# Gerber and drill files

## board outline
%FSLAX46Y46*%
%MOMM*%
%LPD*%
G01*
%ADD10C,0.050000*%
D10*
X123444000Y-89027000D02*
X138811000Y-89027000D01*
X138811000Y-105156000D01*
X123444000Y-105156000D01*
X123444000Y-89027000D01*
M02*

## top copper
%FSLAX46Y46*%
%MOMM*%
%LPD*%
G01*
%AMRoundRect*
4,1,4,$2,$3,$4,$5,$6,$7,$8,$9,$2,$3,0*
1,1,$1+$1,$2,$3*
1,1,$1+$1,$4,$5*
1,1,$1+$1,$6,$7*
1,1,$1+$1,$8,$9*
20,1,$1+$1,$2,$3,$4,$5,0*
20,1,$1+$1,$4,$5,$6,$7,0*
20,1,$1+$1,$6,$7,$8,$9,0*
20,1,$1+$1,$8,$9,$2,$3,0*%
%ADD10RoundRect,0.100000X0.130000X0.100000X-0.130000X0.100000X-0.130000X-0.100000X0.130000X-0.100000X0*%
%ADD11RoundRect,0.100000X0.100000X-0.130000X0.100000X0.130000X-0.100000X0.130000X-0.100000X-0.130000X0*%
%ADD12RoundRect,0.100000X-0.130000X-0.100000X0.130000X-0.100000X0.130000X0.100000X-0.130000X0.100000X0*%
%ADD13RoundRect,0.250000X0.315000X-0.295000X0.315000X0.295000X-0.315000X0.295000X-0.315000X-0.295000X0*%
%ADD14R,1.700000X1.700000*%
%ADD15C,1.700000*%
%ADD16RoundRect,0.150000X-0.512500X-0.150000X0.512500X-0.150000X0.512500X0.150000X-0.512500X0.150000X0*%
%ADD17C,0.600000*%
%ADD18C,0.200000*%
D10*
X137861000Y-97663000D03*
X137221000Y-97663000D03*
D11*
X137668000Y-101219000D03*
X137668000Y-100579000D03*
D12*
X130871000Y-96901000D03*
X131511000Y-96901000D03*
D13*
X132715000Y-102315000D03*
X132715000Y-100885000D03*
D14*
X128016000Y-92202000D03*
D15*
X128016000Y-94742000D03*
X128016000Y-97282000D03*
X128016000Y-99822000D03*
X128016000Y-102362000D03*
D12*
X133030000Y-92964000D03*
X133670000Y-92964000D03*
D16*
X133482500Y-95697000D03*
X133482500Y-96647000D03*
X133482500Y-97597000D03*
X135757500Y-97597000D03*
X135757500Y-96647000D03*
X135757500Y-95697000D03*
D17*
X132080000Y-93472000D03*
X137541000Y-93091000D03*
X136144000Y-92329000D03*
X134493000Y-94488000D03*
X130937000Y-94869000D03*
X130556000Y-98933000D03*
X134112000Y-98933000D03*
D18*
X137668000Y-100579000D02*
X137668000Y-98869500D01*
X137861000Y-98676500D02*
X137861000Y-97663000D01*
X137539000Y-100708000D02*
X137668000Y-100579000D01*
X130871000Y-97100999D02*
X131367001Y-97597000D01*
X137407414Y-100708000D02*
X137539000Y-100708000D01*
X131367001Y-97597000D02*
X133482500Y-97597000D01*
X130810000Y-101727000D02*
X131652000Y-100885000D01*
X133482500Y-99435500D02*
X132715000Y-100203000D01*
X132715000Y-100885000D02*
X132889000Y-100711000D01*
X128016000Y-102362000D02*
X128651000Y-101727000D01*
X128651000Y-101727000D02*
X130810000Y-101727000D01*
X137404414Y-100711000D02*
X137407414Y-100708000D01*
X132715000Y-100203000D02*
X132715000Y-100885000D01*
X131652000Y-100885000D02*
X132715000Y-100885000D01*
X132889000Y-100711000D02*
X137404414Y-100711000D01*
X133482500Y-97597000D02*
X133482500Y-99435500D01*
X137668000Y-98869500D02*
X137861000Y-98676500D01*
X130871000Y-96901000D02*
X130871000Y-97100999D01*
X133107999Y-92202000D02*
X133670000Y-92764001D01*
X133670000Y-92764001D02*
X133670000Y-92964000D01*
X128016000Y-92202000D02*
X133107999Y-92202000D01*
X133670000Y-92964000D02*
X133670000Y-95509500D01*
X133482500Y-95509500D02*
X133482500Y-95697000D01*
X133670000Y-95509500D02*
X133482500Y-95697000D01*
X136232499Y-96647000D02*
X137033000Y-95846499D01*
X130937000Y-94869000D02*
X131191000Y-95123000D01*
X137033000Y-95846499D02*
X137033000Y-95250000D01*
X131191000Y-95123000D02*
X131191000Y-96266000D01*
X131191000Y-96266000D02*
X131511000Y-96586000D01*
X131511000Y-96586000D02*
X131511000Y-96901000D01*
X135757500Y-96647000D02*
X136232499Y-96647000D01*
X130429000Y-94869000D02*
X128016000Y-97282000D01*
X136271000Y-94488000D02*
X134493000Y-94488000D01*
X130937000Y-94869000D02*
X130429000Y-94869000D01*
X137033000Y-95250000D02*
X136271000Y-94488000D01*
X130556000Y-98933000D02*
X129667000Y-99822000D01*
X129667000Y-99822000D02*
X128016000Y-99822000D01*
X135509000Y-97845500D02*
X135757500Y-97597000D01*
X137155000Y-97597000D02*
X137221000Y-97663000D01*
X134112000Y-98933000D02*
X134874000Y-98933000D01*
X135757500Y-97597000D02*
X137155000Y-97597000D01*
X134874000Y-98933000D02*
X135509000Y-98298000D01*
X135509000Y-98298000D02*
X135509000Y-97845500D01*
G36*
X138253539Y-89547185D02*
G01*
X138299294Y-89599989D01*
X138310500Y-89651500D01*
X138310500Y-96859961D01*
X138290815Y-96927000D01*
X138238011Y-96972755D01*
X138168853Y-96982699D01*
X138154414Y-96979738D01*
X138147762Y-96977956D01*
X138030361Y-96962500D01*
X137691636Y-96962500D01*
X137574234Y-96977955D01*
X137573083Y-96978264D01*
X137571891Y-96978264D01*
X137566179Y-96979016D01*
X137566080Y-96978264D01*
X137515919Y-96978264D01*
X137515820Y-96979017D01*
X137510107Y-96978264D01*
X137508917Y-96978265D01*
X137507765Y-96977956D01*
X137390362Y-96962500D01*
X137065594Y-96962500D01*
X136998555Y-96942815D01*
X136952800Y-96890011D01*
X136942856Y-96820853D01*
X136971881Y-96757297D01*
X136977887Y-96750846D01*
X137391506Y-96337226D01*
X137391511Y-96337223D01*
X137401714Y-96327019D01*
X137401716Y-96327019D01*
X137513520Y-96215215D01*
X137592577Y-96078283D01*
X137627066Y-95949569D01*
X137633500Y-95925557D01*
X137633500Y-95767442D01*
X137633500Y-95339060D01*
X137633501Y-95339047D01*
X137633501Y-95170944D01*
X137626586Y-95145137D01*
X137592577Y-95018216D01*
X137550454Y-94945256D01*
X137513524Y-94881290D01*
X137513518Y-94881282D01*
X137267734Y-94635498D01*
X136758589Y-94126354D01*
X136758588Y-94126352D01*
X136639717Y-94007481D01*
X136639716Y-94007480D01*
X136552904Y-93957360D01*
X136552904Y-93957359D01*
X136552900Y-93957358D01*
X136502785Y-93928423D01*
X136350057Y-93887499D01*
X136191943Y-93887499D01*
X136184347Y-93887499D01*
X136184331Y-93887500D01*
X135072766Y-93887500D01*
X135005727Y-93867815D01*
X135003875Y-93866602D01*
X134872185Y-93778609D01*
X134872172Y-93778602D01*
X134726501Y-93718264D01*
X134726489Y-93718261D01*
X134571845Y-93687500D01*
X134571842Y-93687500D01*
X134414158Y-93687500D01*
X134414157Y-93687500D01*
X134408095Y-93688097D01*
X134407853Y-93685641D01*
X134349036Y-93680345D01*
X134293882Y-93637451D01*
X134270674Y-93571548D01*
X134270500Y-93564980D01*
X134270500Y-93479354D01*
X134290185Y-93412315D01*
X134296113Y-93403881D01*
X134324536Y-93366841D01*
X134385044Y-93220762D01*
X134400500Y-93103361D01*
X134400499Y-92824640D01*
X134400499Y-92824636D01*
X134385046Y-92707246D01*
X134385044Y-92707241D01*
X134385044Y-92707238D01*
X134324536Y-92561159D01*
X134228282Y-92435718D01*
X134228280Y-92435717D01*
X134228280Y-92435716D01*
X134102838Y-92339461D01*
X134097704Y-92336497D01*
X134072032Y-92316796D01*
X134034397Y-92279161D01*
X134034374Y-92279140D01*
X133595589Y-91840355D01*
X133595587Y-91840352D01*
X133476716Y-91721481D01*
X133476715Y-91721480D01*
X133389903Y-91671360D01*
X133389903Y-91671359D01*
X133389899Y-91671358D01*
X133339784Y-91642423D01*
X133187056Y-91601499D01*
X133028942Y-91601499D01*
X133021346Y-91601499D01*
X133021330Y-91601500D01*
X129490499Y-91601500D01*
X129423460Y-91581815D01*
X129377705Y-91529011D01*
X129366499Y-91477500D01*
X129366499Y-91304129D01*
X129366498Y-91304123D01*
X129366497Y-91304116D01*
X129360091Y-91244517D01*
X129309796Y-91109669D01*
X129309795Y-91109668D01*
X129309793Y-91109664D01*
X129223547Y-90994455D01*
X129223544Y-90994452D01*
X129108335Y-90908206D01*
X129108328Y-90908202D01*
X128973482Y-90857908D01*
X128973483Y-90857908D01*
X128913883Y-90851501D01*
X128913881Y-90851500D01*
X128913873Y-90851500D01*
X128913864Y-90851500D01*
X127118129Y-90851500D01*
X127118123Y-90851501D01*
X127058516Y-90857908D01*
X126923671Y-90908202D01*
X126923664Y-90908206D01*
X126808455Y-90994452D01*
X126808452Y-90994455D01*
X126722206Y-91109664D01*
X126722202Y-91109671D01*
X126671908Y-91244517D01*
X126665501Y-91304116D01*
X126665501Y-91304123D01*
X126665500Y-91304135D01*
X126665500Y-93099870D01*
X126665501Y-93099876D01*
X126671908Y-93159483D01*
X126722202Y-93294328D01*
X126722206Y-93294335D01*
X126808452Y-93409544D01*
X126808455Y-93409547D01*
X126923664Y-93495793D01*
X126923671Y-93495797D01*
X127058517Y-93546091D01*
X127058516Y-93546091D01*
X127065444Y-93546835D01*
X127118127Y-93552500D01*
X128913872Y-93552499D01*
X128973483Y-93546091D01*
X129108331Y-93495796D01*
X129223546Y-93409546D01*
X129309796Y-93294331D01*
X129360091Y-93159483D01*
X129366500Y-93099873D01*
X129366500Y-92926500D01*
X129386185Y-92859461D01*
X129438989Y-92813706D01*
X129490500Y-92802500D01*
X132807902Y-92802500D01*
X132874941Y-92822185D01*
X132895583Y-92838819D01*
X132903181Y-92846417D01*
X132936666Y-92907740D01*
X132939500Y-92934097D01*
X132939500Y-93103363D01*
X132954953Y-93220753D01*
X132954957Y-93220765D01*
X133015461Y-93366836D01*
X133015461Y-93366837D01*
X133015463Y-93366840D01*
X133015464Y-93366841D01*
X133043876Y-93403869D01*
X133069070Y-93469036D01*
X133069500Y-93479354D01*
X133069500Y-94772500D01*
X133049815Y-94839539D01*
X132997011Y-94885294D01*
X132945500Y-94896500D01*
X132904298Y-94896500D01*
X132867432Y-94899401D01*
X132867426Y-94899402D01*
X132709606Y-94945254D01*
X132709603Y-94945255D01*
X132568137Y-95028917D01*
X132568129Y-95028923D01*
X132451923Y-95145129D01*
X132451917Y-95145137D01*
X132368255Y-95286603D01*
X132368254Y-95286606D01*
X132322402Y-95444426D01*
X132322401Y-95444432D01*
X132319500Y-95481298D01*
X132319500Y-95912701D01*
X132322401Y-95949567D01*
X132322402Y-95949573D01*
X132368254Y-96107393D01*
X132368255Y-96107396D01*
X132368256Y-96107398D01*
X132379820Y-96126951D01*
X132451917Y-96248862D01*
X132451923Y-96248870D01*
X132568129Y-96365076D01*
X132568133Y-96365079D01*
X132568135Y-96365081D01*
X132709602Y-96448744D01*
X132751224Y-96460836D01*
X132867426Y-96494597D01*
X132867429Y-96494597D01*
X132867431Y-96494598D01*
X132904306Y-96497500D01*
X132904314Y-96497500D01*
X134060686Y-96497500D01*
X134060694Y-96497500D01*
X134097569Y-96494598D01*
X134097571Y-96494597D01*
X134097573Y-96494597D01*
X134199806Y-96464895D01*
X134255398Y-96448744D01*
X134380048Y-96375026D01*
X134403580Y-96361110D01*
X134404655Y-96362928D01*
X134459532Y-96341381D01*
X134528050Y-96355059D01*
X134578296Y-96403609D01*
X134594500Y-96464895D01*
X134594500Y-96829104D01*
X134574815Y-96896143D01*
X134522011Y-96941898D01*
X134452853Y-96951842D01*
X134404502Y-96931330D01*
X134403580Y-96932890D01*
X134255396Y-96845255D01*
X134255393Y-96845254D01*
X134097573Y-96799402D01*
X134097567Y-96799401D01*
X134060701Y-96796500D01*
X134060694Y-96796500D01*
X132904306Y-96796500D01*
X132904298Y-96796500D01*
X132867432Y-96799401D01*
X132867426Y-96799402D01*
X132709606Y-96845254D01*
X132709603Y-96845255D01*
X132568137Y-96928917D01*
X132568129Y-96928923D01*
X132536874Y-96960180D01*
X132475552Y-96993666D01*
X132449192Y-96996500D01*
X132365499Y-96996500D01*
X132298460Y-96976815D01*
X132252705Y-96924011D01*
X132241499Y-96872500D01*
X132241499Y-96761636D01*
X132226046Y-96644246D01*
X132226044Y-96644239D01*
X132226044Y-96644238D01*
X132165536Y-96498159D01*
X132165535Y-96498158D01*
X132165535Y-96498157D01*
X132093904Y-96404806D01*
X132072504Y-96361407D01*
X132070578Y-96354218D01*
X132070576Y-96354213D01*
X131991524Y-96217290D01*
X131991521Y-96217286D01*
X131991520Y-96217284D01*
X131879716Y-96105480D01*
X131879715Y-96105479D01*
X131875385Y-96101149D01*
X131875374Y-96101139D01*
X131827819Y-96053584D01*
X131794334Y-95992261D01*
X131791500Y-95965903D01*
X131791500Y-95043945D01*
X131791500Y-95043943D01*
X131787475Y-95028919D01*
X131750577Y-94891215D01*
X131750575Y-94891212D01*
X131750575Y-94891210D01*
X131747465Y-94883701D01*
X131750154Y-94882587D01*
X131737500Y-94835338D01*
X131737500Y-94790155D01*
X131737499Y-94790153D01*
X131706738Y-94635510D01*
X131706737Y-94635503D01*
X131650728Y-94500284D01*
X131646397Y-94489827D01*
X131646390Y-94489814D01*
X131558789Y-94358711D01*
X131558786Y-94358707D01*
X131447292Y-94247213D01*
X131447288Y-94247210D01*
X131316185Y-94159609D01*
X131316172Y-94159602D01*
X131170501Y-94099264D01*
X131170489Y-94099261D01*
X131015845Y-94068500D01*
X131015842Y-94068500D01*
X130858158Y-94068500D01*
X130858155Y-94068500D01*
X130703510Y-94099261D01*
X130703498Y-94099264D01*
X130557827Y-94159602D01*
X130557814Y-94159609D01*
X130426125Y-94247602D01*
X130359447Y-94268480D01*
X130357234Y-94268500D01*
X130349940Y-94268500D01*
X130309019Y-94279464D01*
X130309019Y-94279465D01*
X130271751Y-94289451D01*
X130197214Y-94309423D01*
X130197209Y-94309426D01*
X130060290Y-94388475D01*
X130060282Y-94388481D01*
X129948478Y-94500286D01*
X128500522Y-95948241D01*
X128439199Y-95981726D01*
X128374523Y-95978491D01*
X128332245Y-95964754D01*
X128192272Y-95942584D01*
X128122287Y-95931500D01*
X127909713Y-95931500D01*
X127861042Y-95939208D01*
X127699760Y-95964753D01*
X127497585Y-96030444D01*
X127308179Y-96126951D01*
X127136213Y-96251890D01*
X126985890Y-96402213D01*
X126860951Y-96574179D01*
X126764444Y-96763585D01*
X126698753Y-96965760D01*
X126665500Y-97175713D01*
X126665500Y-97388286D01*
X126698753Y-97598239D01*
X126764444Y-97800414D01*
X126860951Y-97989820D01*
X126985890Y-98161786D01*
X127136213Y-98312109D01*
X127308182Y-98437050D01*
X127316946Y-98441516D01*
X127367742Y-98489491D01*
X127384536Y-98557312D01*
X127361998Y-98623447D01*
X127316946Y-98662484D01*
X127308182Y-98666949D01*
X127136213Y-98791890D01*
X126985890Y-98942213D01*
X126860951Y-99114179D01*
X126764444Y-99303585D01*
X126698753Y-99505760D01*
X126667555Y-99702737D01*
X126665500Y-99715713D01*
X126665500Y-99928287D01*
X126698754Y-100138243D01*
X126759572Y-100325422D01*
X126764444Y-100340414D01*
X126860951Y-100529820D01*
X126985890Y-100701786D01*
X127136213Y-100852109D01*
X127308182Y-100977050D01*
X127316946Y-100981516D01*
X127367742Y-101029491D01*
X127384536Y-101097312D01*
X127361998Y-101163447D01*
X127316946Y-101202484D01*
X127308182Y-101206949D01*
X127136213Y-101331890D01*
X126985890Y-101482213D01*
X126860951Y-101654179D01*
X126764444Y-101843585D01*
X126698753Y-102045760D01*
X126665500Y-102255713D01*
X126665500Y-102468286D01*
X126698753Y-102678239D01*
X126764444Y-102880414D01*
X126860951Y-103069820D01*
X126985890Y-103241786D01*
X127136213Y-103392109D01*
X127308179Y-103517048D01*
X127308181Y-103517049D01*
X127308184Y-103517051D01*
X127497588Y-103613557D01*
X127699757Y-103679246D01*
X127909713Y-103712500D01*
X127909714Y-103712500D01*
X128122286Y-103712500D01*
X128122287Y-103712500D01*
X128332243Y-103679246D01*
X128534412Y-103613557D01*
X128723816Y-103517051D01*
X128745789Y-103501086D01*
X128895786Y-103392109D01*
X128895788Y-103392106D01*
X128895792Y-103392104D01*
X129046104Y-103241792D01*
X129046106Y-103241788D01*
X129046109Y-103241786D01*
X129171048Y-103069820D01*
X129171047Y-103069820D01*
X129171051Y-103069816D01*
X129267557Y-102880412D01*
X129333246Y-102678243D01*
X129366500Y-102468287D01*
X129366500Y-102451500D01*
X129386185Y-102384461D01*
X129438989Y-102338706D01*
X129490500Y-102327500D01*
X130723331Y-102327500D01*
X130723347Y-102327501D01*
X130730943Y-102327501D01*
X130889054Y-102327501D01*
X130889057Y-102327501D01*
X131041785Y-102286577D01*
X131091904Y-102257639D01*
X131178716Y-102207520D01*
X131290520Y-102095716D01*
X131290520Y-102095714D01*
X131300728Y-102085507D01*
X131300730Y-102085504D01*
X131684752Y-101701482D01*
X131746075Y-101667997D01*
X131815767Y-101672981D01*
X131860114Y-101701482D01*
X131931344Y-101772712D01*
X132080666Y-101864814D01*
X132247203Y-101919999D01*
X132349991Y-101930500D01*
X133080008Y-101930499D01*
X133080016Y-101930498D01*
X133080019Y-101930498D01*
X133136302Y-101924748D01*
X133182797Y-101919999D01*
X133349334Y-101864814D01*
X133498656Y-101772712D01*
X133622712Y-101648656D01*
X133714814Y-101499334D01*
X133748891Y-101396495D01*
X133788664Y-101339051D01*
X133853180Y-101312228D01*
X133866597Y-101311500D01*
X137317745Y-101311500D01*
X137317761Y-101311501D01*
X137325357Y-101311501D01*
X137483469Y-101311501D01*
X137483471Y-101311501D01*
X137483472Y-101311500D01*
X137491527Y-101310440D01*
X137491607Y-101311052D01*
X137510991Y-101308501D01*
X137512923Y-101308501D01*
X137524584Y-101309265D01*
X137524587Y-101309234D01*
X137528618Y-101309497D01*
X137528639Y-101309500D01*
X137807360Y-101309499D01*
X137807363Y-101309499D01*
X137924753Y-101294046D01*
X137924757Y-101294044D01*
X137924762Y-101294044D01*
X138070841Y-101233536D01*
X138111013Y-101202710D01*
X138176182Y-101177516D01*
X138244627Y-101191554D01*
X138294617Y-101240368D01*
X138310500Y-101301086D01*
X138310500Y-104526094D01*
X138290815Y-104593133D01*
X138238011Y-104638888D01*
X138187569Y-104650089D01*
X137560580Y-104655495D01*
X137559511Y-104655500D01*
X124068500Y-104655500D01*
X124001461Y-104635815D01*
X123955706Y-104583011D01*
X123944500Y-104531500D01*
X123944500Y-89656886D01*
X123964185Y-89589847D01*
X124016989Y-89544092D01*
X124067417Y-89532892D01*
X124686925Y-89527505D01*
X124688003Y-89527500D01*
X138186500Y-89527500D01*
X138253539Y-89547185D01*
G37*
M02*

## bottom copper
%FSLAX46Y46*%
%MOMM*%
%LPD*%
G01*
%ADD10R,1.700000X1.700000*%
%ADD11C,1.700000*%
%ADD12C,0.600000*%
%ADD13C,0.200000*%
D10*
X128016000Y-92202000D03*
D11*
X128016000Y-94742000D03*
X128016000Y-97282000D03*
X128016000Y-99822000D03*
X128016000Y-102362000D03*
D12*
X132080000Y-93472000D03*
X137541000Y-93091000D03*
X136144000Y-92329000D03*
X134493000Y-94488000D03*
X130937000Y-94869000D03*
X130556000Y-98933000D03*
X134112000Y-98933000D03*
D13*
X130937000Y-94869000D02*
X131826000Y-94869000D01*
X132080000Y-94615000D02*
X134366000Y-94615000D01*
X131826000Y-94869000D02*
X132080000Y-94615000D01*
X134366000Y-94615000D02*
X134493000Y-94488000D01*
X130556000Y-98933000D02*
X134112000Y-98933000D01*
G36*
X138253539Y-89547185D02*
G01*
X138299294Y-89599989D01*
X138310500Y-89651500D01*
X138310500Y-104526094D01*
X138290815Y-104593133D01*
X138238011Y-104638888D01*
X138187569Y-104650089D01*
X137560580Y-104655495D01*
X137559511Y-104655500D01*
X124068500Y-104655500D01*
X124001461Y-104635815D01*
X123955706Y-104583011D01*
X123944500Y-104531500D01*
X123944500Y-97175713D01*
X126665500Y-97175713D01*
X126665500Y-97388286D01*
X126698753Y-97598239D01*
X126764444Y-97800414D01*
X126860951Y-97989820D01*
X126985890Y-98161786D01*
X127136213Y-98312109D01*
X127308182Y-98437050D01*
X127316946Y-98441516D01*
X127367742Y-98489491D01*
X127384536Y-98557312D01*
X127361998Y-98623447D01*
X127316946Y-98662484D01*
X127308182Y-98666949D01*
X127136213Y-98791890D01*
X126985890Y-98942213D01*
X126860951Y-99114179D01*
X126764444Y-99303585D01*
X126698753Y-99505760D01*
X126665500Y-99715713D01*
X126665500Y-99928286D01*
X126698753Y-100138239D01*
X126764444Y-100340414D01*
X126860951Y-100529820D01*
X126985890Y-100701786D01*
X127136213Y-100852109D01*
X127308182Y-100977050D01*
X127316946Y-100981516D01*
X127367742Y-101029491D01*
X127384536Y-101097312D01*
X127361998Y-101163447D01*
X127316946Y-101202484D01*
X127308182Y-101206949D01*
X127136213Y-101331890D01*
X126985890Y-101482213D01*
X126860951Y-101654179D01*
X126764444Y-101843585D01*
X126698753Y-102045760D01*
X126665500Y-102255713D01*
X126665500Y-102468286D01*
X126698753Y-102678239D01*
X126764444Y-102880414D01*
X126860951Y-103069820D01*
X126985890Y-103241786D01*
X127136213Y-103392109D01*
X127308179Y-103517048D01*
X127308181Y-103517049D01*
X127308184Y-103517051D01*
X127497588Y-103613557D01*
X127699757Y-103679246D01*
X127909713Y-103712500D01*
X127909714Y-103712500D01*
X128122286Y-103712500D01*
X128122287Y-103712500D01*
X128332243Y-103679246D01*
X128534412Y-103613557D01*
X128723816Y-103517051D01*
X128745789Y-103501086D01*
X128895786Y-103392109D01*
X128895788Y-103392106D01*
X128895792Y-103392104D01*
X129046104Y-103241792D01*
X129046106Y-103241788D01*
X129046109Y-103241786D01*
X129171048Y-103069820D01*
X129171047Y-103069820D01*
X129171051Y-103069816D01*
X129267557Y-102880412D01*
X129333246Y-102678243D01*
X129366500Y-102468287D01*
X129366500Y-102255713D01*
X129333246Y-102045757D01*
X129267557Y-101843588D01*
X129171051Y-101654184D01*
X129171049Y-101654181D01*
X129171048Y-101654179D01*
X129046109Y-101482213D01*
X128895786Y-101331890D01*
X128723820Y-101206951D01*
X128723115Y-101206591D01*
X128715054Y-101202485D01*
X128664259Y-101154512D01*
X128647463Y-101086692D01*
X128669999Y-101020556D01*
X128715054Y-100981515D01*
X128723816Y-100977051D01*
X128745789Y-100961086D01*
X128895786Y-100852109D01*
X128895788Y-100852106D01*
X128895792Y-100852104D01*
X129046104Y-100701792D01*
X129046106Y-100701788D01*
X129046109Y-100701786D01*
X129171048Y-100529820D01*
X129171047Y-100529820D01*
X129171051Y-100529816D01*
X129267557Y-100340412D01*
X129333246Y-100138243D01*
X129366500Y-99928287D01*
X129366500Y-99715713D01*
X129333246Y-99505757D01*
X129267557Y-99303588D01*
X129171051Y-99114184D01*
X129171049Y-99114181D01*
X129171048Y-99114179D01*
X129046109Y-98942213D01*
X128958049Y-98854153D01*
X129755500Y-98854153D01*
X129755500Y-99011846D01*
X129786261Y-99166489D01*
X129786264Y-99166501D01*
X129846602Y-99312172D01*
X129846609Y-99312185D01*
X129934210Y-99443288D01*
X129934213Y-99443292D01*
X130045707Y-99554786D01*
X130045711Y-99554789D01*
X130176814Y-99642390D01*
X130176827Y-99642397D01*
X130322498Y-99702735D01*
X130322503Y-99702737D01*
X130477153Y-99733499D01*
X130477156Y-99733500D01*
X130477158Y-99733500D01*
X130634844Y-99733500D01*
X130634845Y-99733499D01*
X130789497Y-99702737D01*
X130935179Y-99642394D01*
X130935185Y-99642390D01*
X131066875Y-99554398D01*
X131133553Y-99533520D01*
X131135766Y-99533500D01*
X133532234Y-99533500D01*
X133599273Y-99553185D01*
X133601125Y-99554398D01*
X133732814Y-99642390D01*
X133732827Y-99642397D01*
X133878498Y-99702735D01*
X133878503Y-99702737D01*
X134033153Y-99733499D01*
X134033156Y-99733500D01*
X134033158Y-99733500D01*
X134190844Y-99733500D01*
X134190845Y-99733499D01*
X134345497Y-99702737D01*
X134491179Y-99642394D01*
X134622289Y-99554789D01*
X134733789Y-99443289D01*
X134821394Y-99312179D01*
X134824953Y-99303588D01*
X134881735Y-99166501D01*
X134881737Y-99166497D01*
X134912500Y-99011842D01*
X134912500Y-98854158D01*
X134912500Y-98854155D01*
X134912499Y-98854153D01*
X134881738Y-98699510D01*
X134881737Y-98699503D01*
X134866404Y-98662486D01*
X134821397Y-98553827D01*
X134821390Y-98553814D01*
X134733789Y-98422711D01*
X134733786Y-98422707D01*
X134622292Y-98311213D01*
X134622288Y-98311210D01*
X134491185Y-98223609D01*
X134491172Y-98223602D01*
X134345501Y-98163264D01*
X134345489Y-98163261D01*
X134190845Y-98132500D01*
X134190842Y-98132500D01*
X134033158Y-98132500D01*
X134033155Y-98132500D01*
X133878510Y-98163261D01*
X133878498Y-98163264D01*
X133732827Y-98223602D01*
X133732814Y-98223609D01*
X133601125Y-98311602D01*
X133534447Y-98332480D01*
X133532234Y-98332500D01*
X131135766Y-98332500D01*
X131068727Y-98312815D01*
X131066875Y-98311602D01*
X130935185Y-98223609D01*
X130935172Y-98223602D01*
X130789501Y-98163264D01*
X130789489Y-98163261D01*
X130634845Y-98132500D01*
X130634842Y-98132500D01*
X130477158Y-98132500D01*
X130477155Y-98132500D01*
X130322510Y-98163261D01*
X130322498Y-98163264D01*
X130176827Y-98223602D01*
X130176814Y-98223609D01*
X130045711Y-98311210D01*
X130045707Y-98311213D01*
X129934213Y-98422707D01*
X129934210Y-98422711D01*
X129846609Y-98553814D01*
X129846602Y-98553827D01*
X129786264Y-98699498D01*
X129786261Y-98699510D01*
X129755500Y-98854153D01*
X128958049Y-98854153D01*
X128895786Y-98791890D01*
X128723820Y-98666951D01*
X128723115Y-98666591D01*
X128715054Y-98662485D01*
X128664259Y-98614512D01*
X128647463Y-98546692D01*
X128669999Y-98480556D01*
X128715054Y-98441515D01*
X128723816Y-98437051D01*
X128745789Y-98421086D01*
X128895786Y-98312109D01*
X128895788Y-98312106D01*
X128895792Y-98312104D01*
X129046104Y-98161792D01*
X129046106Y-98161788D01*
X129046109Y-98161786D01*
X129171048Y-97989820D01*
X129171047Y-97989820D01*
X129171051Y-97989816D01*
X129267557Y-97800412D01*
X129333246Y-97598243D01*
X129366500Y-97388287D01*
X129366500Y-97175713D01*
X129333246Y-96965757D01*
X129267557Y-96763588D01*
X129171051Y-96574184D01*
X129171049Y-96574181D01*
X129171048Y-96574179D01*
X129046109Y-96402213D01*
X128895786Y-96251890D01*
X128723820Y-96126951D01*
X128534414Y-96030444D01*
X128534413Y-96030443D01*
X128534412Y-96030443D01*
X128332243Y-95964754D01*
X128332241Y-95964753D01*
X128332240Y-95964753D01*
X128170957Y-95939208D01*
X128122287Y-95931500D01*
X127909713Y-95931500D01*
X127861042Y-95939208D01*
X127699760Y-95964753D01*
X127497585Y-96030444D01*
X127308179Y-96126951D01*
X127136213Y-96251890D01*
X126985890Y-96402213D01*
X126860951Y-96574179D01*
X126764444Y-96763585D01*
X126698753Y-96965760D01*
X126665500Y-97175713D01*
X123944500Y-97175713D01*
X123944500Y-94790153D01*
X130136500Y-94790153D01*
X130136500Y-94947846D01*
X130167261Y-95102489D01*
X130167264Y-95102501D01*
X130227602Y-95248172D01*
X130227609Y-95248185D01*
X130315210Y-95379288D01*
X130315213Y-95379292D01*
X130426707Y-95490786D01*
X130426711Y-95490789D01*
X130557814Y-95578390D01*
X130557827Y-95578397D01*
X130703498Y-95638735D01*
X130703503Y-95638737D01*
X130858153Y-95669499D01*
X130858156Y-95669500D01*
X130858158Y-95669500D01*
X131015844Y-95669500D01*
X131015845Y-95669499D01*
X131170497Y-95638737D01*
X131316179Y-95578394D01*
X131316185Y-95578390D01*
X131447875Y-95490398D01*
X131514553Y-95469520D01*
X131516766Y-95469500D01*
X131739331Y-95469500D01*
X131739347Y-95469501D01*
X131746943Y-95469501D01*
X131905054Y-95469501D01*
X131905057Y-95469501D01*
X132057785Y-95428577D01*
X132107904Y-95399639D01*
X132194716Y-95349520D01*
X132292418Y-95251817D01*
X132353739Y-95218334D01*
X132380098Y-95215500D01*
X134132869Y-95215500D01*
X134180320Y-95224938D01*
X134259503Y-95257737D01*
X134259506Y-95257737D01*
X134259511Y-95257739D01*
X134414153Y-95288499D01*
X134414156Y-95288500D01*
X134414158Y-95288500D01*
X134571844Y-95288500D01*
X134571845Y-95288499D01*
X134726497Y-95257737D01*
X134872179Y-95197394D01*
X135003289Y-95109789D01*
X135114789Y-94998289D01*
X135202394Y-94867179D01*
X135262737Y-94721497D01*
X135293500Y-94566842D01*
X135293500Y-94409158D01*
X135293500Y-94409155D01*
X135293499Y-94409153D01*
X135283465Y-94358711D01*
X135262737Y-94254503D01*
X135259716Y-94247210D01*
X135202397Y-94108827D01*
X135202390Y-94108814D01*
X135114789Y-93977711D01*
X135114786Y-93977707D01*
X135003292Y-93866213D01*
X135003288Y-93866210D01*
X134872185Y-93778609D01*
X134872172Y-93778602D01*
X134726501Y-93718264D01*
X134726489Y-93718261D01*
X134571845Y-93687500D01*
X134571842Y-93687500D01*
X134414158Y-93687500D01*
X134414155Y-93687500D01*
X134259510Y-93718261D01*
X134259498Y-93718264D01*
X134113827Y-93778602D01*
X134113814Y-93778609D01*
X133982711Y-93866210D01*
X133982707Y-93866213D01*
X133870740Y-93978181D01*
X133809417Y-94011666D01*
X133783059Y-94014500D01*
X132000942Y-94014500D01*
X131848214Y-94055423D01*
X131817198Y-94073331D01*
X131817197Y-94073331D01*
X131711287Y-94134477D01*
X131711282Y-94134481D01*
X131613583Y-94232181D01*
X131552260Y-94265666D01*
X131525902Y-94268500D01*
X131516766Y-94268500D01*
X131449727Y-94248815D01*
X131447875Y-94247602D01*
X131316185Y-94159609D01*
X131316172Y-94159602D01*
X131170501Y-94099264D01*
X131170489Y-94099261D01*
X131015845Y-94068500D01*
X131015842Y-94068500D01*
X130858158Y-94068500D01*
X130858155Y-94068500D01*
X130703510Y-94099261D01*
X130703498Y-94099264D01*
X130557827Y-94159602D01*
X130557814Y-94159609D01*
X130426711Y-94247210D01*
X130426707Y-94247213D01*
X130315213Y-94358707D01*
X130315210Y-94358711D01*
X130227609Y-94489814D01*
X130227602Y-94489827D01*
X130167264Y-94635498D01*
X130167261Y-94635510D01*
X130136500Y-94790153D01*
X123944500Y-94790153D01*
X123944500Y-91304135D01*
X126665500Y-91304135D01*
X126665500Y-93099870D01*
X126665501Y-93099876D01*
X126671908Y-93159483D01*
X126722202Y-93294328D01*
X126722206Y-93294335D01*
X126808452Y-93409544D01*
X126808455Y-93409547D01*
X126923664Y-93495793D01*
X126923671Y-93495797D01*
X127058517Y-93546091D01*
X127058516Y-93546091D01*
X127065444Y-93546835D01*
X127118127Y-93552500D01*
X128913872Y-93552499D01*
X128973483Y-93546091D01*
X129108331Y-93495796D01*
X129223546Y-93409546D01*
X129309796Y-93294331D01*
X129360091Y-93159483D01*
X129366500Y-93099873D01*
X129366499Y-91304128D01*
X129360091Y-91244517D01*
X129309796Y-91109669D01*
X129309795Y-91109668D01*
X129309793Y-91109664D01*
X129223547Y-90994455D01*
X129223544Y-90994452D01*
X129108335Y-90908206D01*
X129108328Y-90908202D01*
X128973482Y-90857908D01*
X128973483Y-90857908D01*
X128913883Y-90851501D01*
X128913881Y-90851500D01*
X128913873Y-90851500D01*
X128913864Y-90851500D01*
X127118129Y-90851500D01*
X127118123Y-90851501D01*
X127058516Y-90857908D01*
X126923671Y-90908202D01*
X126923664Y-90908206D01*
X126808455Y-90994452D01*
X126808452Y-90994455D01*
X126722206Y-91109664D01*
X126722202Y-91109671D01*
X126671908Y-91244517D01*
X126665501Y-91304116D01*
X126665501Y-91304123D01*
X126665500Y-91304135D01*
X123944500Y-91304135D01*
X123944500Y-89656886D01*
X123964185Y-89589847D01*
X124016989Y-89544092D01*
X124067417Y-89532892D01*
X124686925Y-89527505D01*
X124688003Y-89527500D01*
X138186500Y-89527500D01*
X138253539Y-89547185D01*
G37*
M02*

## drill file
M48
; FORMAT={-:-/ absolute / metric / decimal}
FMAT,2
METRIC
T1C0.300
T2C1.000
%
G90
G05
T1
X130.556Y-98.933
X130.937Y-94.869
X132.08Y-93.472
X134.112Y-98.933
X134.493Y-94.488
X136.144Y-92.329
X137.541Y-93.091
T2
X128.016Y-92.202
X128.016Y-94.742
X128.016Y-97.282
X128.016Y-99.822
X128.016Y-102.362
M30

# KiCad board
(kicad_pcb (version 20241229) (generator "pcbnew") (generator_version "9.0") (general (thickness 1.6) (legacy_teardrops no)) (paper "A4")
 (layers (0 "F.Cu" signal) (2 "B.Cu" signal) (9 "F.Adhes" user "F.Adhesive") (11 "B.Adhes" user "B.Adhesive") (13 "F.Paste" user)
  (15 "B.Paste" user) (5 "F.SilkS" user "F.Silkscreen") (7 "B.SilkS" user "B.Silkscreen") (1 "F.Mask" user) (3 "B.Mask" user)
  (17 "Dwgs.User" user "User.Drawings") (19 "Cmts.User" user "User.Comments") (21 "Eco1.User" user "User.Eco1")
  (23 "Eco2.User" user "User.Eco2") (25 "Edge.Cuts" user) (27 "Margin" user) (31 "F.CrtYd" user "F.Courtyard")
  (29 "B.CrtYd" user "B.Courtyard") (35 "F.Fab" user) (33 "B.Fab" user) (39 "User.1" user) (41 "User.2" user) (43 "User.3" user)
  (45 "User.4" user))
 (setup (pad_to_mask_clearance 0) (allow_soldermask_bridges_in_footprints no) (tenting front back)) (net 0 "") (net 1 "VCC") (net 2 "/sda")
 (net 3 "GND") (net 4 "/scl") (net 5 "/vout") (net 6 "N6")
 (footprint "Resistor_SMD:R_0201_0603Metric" (layer "F.Cu") (at 137.541 97.663 180)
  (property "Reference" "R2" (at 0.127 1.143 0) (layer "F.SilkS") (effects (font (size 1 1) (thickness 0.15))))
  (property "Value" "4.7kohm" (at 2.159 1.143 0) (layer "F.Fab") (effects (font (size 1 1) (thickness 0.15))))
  (pad "" smd roundrect (at -0.345 0 180) (size 0.318 0.36) (layers "F.Paste") (roundrect_rratio 0.25))
  (pad "" smd roundrect (at 0.345 0 180) (size 0.318 0.36) (layers "F.Paste") (roundrect_rratio 0.25))
  (pad "1" smd roundrect (at -0.32 0 180) (size 0.46 0.4) (layers "F.Cu" "F.Mask") (roundrect_rratio 0.25) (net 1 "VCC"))
  (pad "2" smd roundrect (at 0.32 0 180) (size 0.46 0.4) (layers "F.Cu" "F.Mask") (roundrect_rratio 0.25) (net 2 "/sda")))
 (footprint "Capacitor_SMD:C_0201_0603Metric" (layer "F.Cu") (at 137.668 100.899 90)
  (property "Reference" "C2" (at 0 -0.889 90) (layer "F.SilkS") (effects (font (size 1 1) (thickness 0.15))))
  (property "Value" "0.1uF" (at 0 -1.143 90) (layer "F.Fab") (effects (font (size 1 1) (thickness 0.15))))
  (pad "" smd roundrect (at -0.345 0 90) (size 0.318 0.36) (layers "F.Paste") (roundrect_rratio 0.25))
  (pad "" smd roundrect (at 0.345 0 90) (size 0.318 0.36) (layers "F.Paste") (roundrect_rratio 0.25))
  (pad "1" smd roundrect (at -0.32 0 90) (size 0.46 0.4) (layers "F.Cu" "F.Mask") (roundrect_rratio 0.25) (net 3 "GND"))
  (pad "2" smd roundrect (at 0.32 0 90) (size 0.46 0.4) (layers "F.Cu" "F.Mask") (roundrect_rratio 0.25) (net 1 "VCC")))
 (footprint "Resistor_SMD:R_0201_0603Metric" (layer "F.Cu") (at 131.191 96.901)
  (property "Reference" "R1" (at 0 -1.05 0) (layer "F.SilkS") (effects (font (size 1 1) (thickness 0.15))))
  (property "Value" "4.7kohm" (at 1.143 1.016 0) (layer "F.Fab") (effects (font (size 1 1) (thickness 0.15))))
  (pad "" smd roundrect (at -0.345 0) (size 0.318 0.36) (layers "F.Paste") (roundrect_rratio 0.25))
  (pad "" smd roundrect (at 0.345 0) (size 0.318 0.36) (layers "F.Paste") (roundrect_rratio 0.25))
  (pad "1" smd roundrect (at -0.32 0) (size 0.46 0.4) (layers "F.Cu" "F.Mask") (roundrect_rratio 0.25) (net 1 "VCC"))
  (pad "2" smd roundrect (at 0.32 0) (size 0.46 0.4) (layers "F.Cu" "F.Mask") (roundrect_rratio 0.25) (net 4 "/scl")))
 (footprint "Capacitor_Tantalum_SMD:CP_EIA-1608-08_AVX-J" (layer "F.Cu") (at 132.715 101.6 90)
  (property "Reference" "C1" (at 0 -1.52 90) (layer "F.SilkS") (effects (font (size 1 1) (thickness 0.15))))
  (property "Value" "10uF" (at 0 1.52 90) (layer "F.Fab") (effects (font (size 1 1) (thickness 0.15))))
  (pad "1" smd roundrect (at -0.715 0 90) (size 1.09 1.13) (layers "F.Cu" "F.Mask" "F.Paste") (roundrect_rratio 0.229358) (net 3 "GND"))
  (pad "2" smd roundrect (at 0.715 0 90) (size 1.09 1.13) (layers "F.Cu" "F.Mask" "F.Paste") (roundrect_rratio 0.229358) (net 1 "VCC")))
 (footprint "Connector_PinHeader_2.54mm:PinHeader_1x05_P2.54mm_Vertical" (layer "F.Cu") (at 128.016 92.202)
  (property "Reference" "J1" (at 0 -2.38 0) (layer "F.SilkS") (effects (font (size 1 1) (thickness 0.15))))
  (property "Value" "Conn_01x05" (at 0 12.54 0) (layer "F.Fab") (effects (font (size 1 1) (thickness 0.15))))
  (pad "1" thru_hole rect (at 0 0) (size 1.7 1.7) (drill 1) (layers "*.Cu" "*.Mask") (remove_unused_layers no) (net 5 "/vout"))
  (pad "2" thru_hole circle (at 0 2.54) (size 1.7 1.7) (drill 1) (layers "*.Cu" "*.Mask") (remove_unused_layers no) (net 3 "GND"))
  (pad "3" thru_hole circle (at 0 5.08) (size 1.7 1.7) (drill 1) (layers "*.Cu" "*.Mask") (remove_unused_layers no) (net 4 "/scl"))
  (pad "4" thru_hole circle (at 0 7.62) (size 1.7 1.7) (drill 1) (layers "*.Cu" "*.Mask") (remove_unused_layers no) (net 2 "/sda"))
  (pad "5" thru_hole circle (at 0 10.16) (size 1.7 1.7) (drill 1) (layers "*.Cu" "*.Mask") (remove_unused_layers no) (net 1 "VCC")))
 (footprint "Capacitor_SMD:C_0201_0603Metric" (layer "F.Cu") (at 133.35 92.964)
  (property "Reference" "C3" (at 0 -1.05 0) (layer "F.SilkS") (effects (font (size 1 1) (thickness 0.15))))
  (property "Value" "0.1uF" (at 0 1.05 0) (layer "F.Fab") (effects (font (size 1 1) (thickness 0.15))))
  (pad "" smd roundrect (at -0.345 0) (size 0.318 0.36) (layers "F.Paste") (roundrect_rratio 0.25))
  (pad "" smd roundrect (at 0.345 0) (size 0.318 0.36) (layers "F.Paste") (roundrect_rratio 0.25))
  (pad "1" smd roundrect (at -0.32 0) (size 0.46 0.4) (layers "F.Cu" "F.Mask") (roundrect_rratio 0.25) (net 3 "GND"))
  (pad "2" smd roundrect (at 0.32 0) (size 0.46 0.4) (layers "F.Cu" "F.Mask") (roundrect_rratio 0.25) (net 5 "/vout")))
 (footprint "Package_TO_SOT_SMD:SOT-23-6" (layer "F.Cu") (at 134.62 96.647)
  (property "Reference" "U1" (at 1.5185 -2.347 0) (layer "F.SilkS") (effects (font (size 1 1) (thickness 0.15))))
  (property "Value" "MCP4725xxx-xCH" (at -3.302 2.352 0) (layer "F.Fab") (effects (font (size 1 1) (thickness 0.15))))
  (pad "1" smd roundrect (at -1.1375 -0.95) (size 1.325 0.6) (layers "F.Cu" "F.Mask" "F.Paste") (roundrect_rratio 0.25) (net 5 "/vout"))
  (pad "2" smd roundrect (at -1.1375 0) (size 1.325 0.6) (layers "F.Cu" "F.Mask" "F.Paste") (roundrect_rratio 0.25) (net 3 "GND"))
  (pad "3" smd roundrect (at -1.1375 0.95) (size 1.325 0.6) (layers "F.Cu" "F.Mask" "F.Paste") (roundrect_rratio 0.25) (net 1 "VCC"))
  (pad "4" smd roundrect (at 1.1375 0.95) (size 1.325 0.6) (layers "F.Cu" "F.Mask" "F.Paste") (roundrect_rratio 0.25) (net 2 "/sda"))
  (pad "5" smd roundrect (at 1.1375 0) (size 1.325 0.6) (layers "F.Cu" "F.Mask" "F.Paste") (roundrect_rratio 0.25) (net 4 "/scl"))
  (pad "6" smd roundrect (at 1.1375 -0.95) (size 1.325 0.6) (layers "F.Cu" "F.Mask" "F.Paste") (roundrect_rratio 0.25) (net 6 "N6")))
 (gr_rect (start 123.444 89.027) (end 138.811 105.156) (stroke (width 0.05) (type default)) (fill no) (layer "Edge.Cuts"))
 (via (at 132.08 93.472) (size 0.6) (drill 0.3) (layers "F.Cu" "B.Cu") (free yes) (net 3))
 (via (at 137.541 93.091) (size 0.6) (drill 0.3) (layers "F.Cu" "B.Cu") (free yes) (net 3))
 (via (at 136.144 92.329) (size 0.6) (drill 0.3) (layers "F.Cu" "B.Cu") (free yes) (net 3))
 (segment (start 137.668 100.579) (end 137.668 98.8695) (width 0.2) (layer "F.Cu") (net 1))
 (segment (start 137.861 98.6765) (end 137.861 97.663) (width 0.2) (layer "F.Cu") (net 1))
 (segment (start 137.539 100.708) (end 137.668 100.579) (width 0.2) (layer "F.Cu") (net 1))
 (segment (start 130.871 97.100999) (end 131.367001 97.597) (width 0.2) (layer "F.Cu") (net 1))
 (segment (start 137.407414 100.708) (end 137.539 100.708) (width 0.2) (layer "F.Cu") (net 1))
 (segment (start 131.367001 97.597) (end 133.4825 97.597) (width 0.2) (layer "F.Cu") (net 1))
 (segment (start 130.81 101.727) (end 131.652 100.885) (width 0.2) (layer "F.Cu") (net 1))
 (segment (start 133.4825 99.4355) (end 132.715 100.203) (width 0.2) (layer "F.Cu") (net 1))
 (segment (start 132.715 100.885) (end 132.889 100.711) (width 0.2) (layer "F.Cu") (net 1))
 (segment (start 128.016 102.362) (end 128.651 101.727) (width 0.2) (layer "F.Cu") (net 1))
 (segment (start 128.651 101.727) (end 130.81 101.727) (width 0.2) (layer "F.Cu") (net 1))
 (segment (start 137.404414 100.711) (end 137.407414 100.708) (width 0.2) (layer "F.Cu") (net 1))
 (segment (start 132.715 100.203) (end 132.715 100.885) (width 0.2) (layer "F.Cu") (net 1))
 (segment (start 131.652 100.885) (end 132.715 100.885) (width 0.2) (layer "F.Cu") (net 1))
 (segment (start 132.889 100.711) (end 137.404414 100.711) (width 0.2) (layer "F.Cu") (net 1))
 (segment (start 133.4825 97.597) (end 133.4825 99.4355) (width 0.2) (layer "F.Cu") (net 1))
 (segment (start 137.668 98.8695) (end 137.861 98.6765) (width 0.2) (layer "F.Cu") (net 1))
 (segment (start 130.871 96.901) (end 130.871 97.100999) (width 0.2) (layer "F.Cu") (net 1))
 (segment (start 133.107999 92.202) (end 133.67 92.764001) (width 0.2) (layer "F.Cu") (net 5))
 (segment (start 133.67 92.764001) (end 133.67 92.964) (width 0.2) (layer "F.Cu") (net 5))
 (segment (start 128.016 92.202) (end 133.107999 92.202) (width 0.2) (layer "F.Cu") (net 5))
 (segment (start 133.67 92.964) (end 133.67 95.5095) (width 0.2) (layer "F.Cu") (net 5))
 (segment (start 133.4825 95.5095) (end 133.4825 95.697) (width 0.2) (layer "F.Cu") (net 5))
 (segment (start 133.67 95.5095) (end 133.4825 95.697) (width 0.2) (layer "F.Cu") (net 5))
 (segment (start 136.232499 96.647) (end 137.033 95.846499) (width 0.2) (layer "F.Cu") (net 4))
 (segment (start 130.937 94.869) (end 131.191 95.123) (width 0.2) (layer "F.Cu") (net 4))
 (segment (start 137.033 95.846499) (end 137.033 95.25) (width 0.2) (layer "F.Cu") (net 4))
 (segment (start 131.191 95.123) (end 131.191 96.266) (width 0.2) (layer "F.Cu") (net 4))
 (segment (start 131.191 96.266) (end 131.511 96.586) (width 0.2) (layer "F.Cu") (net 4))
 (segment (start 131.511 96.586) (end 131.511 96.901) (width 0.2) (layer "F.Cu") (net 4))
 (segment (start 135.7575 96.647) (end 136.232499 96.647) (width 0.2) (layer "F.Cu") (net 4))
 (segment (start 130.429 94.869) (end 128.016 97.282) (width 0.2) (layer "F.Cu") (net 4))
 (segment (start 136.271 94.488) (end 134.493 94.488) (width 0.2) (layer "F.Cu") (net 4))
 (segment (start 130.937 94.869) (end 130.429 94.869) (width 0.2) (layer "F.Cu") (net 4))
 (segment (start 137.033 95.25) (end 136.271 94.488) (width 0.2) (layer "F.Cu") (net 4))
 (via (at 134.493 94.488) (size 0.6) (drill 0.3) (layers "F.Cu" "B.Cu") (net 4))
 (via (at 130.937 94.869) (size 0.6) (drill 0.3) (layers "F.Cu" "B.Cu") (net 4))
 (segment (start 130.937 94.869) (end 131.826 94.869) (width 0.2) (layer "B.Cu") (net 4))
 (segment (start 132.08 94.615) (end 134.366 94.615) (width 0.2) (layer "B.Cu") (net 4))
 (segment (start 131.826 94.869) (end 132.08 94.615) (width 0.2) (layer "B.Cu") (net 4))
 (segment (start 134.366 94.615) (end 134.493 94.488) (width 0.2) (layer "B.Cu") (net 4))
 (segment (start 130.556 98.933) (end 129.667 99.822) (width 0.2) (layer "F.Cu") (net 2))
 (segment (start 129.667 99.822) (end 128.016 99.822) (width 0.2) (layer "F.Cu") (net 2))
 (segment (start 135.509 97.8455) (end 135.7575 97.597) (width 0.2) (layer "F.Cu") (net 2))
 (segment (start 137.155 97.597) (end 137.221 97.663) (width 0.2) (layer "F.Cu") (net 2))
 (segment (start 134.112 98.933) (end 134.874 98.933) (width 0.2) (layer "F.Cu") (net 2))
 (segment (start 135.7575 97.597) (end 137.155 97.597) (width 0.2) (layer "F.Cu") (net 2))
 (segment (start 134.874 98.933) (end 135.509 98.298) (width 0.2) (layer "F.Cu") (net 2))
 (segment (start 135.509 98.298) (end 135.509 97.8455) (width 0.2) (layer "F.Cu") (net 2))
 (via (at 130.556 98.933) (size 0.6) (drill 0.3) (layers "F.Cu" "B.Cu") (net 2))
 (via (at 134.112 98.933) (size 0.6) (drill 0.3) (layers "F.Cu" "B.Cu") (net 2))
 (segment (start 130.556 98.933) (end 134.112 98.933) (width 0.2) (layer "B.Cu") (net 2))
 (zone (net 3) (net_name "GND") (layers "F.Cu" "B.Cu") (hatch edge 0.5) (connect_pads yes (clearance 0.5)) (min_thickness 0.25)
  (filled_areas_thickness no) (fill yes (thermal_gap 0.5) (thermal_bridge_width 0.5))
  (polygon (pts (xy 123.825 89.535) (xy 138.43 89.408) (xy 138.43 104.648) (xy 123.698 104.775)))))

